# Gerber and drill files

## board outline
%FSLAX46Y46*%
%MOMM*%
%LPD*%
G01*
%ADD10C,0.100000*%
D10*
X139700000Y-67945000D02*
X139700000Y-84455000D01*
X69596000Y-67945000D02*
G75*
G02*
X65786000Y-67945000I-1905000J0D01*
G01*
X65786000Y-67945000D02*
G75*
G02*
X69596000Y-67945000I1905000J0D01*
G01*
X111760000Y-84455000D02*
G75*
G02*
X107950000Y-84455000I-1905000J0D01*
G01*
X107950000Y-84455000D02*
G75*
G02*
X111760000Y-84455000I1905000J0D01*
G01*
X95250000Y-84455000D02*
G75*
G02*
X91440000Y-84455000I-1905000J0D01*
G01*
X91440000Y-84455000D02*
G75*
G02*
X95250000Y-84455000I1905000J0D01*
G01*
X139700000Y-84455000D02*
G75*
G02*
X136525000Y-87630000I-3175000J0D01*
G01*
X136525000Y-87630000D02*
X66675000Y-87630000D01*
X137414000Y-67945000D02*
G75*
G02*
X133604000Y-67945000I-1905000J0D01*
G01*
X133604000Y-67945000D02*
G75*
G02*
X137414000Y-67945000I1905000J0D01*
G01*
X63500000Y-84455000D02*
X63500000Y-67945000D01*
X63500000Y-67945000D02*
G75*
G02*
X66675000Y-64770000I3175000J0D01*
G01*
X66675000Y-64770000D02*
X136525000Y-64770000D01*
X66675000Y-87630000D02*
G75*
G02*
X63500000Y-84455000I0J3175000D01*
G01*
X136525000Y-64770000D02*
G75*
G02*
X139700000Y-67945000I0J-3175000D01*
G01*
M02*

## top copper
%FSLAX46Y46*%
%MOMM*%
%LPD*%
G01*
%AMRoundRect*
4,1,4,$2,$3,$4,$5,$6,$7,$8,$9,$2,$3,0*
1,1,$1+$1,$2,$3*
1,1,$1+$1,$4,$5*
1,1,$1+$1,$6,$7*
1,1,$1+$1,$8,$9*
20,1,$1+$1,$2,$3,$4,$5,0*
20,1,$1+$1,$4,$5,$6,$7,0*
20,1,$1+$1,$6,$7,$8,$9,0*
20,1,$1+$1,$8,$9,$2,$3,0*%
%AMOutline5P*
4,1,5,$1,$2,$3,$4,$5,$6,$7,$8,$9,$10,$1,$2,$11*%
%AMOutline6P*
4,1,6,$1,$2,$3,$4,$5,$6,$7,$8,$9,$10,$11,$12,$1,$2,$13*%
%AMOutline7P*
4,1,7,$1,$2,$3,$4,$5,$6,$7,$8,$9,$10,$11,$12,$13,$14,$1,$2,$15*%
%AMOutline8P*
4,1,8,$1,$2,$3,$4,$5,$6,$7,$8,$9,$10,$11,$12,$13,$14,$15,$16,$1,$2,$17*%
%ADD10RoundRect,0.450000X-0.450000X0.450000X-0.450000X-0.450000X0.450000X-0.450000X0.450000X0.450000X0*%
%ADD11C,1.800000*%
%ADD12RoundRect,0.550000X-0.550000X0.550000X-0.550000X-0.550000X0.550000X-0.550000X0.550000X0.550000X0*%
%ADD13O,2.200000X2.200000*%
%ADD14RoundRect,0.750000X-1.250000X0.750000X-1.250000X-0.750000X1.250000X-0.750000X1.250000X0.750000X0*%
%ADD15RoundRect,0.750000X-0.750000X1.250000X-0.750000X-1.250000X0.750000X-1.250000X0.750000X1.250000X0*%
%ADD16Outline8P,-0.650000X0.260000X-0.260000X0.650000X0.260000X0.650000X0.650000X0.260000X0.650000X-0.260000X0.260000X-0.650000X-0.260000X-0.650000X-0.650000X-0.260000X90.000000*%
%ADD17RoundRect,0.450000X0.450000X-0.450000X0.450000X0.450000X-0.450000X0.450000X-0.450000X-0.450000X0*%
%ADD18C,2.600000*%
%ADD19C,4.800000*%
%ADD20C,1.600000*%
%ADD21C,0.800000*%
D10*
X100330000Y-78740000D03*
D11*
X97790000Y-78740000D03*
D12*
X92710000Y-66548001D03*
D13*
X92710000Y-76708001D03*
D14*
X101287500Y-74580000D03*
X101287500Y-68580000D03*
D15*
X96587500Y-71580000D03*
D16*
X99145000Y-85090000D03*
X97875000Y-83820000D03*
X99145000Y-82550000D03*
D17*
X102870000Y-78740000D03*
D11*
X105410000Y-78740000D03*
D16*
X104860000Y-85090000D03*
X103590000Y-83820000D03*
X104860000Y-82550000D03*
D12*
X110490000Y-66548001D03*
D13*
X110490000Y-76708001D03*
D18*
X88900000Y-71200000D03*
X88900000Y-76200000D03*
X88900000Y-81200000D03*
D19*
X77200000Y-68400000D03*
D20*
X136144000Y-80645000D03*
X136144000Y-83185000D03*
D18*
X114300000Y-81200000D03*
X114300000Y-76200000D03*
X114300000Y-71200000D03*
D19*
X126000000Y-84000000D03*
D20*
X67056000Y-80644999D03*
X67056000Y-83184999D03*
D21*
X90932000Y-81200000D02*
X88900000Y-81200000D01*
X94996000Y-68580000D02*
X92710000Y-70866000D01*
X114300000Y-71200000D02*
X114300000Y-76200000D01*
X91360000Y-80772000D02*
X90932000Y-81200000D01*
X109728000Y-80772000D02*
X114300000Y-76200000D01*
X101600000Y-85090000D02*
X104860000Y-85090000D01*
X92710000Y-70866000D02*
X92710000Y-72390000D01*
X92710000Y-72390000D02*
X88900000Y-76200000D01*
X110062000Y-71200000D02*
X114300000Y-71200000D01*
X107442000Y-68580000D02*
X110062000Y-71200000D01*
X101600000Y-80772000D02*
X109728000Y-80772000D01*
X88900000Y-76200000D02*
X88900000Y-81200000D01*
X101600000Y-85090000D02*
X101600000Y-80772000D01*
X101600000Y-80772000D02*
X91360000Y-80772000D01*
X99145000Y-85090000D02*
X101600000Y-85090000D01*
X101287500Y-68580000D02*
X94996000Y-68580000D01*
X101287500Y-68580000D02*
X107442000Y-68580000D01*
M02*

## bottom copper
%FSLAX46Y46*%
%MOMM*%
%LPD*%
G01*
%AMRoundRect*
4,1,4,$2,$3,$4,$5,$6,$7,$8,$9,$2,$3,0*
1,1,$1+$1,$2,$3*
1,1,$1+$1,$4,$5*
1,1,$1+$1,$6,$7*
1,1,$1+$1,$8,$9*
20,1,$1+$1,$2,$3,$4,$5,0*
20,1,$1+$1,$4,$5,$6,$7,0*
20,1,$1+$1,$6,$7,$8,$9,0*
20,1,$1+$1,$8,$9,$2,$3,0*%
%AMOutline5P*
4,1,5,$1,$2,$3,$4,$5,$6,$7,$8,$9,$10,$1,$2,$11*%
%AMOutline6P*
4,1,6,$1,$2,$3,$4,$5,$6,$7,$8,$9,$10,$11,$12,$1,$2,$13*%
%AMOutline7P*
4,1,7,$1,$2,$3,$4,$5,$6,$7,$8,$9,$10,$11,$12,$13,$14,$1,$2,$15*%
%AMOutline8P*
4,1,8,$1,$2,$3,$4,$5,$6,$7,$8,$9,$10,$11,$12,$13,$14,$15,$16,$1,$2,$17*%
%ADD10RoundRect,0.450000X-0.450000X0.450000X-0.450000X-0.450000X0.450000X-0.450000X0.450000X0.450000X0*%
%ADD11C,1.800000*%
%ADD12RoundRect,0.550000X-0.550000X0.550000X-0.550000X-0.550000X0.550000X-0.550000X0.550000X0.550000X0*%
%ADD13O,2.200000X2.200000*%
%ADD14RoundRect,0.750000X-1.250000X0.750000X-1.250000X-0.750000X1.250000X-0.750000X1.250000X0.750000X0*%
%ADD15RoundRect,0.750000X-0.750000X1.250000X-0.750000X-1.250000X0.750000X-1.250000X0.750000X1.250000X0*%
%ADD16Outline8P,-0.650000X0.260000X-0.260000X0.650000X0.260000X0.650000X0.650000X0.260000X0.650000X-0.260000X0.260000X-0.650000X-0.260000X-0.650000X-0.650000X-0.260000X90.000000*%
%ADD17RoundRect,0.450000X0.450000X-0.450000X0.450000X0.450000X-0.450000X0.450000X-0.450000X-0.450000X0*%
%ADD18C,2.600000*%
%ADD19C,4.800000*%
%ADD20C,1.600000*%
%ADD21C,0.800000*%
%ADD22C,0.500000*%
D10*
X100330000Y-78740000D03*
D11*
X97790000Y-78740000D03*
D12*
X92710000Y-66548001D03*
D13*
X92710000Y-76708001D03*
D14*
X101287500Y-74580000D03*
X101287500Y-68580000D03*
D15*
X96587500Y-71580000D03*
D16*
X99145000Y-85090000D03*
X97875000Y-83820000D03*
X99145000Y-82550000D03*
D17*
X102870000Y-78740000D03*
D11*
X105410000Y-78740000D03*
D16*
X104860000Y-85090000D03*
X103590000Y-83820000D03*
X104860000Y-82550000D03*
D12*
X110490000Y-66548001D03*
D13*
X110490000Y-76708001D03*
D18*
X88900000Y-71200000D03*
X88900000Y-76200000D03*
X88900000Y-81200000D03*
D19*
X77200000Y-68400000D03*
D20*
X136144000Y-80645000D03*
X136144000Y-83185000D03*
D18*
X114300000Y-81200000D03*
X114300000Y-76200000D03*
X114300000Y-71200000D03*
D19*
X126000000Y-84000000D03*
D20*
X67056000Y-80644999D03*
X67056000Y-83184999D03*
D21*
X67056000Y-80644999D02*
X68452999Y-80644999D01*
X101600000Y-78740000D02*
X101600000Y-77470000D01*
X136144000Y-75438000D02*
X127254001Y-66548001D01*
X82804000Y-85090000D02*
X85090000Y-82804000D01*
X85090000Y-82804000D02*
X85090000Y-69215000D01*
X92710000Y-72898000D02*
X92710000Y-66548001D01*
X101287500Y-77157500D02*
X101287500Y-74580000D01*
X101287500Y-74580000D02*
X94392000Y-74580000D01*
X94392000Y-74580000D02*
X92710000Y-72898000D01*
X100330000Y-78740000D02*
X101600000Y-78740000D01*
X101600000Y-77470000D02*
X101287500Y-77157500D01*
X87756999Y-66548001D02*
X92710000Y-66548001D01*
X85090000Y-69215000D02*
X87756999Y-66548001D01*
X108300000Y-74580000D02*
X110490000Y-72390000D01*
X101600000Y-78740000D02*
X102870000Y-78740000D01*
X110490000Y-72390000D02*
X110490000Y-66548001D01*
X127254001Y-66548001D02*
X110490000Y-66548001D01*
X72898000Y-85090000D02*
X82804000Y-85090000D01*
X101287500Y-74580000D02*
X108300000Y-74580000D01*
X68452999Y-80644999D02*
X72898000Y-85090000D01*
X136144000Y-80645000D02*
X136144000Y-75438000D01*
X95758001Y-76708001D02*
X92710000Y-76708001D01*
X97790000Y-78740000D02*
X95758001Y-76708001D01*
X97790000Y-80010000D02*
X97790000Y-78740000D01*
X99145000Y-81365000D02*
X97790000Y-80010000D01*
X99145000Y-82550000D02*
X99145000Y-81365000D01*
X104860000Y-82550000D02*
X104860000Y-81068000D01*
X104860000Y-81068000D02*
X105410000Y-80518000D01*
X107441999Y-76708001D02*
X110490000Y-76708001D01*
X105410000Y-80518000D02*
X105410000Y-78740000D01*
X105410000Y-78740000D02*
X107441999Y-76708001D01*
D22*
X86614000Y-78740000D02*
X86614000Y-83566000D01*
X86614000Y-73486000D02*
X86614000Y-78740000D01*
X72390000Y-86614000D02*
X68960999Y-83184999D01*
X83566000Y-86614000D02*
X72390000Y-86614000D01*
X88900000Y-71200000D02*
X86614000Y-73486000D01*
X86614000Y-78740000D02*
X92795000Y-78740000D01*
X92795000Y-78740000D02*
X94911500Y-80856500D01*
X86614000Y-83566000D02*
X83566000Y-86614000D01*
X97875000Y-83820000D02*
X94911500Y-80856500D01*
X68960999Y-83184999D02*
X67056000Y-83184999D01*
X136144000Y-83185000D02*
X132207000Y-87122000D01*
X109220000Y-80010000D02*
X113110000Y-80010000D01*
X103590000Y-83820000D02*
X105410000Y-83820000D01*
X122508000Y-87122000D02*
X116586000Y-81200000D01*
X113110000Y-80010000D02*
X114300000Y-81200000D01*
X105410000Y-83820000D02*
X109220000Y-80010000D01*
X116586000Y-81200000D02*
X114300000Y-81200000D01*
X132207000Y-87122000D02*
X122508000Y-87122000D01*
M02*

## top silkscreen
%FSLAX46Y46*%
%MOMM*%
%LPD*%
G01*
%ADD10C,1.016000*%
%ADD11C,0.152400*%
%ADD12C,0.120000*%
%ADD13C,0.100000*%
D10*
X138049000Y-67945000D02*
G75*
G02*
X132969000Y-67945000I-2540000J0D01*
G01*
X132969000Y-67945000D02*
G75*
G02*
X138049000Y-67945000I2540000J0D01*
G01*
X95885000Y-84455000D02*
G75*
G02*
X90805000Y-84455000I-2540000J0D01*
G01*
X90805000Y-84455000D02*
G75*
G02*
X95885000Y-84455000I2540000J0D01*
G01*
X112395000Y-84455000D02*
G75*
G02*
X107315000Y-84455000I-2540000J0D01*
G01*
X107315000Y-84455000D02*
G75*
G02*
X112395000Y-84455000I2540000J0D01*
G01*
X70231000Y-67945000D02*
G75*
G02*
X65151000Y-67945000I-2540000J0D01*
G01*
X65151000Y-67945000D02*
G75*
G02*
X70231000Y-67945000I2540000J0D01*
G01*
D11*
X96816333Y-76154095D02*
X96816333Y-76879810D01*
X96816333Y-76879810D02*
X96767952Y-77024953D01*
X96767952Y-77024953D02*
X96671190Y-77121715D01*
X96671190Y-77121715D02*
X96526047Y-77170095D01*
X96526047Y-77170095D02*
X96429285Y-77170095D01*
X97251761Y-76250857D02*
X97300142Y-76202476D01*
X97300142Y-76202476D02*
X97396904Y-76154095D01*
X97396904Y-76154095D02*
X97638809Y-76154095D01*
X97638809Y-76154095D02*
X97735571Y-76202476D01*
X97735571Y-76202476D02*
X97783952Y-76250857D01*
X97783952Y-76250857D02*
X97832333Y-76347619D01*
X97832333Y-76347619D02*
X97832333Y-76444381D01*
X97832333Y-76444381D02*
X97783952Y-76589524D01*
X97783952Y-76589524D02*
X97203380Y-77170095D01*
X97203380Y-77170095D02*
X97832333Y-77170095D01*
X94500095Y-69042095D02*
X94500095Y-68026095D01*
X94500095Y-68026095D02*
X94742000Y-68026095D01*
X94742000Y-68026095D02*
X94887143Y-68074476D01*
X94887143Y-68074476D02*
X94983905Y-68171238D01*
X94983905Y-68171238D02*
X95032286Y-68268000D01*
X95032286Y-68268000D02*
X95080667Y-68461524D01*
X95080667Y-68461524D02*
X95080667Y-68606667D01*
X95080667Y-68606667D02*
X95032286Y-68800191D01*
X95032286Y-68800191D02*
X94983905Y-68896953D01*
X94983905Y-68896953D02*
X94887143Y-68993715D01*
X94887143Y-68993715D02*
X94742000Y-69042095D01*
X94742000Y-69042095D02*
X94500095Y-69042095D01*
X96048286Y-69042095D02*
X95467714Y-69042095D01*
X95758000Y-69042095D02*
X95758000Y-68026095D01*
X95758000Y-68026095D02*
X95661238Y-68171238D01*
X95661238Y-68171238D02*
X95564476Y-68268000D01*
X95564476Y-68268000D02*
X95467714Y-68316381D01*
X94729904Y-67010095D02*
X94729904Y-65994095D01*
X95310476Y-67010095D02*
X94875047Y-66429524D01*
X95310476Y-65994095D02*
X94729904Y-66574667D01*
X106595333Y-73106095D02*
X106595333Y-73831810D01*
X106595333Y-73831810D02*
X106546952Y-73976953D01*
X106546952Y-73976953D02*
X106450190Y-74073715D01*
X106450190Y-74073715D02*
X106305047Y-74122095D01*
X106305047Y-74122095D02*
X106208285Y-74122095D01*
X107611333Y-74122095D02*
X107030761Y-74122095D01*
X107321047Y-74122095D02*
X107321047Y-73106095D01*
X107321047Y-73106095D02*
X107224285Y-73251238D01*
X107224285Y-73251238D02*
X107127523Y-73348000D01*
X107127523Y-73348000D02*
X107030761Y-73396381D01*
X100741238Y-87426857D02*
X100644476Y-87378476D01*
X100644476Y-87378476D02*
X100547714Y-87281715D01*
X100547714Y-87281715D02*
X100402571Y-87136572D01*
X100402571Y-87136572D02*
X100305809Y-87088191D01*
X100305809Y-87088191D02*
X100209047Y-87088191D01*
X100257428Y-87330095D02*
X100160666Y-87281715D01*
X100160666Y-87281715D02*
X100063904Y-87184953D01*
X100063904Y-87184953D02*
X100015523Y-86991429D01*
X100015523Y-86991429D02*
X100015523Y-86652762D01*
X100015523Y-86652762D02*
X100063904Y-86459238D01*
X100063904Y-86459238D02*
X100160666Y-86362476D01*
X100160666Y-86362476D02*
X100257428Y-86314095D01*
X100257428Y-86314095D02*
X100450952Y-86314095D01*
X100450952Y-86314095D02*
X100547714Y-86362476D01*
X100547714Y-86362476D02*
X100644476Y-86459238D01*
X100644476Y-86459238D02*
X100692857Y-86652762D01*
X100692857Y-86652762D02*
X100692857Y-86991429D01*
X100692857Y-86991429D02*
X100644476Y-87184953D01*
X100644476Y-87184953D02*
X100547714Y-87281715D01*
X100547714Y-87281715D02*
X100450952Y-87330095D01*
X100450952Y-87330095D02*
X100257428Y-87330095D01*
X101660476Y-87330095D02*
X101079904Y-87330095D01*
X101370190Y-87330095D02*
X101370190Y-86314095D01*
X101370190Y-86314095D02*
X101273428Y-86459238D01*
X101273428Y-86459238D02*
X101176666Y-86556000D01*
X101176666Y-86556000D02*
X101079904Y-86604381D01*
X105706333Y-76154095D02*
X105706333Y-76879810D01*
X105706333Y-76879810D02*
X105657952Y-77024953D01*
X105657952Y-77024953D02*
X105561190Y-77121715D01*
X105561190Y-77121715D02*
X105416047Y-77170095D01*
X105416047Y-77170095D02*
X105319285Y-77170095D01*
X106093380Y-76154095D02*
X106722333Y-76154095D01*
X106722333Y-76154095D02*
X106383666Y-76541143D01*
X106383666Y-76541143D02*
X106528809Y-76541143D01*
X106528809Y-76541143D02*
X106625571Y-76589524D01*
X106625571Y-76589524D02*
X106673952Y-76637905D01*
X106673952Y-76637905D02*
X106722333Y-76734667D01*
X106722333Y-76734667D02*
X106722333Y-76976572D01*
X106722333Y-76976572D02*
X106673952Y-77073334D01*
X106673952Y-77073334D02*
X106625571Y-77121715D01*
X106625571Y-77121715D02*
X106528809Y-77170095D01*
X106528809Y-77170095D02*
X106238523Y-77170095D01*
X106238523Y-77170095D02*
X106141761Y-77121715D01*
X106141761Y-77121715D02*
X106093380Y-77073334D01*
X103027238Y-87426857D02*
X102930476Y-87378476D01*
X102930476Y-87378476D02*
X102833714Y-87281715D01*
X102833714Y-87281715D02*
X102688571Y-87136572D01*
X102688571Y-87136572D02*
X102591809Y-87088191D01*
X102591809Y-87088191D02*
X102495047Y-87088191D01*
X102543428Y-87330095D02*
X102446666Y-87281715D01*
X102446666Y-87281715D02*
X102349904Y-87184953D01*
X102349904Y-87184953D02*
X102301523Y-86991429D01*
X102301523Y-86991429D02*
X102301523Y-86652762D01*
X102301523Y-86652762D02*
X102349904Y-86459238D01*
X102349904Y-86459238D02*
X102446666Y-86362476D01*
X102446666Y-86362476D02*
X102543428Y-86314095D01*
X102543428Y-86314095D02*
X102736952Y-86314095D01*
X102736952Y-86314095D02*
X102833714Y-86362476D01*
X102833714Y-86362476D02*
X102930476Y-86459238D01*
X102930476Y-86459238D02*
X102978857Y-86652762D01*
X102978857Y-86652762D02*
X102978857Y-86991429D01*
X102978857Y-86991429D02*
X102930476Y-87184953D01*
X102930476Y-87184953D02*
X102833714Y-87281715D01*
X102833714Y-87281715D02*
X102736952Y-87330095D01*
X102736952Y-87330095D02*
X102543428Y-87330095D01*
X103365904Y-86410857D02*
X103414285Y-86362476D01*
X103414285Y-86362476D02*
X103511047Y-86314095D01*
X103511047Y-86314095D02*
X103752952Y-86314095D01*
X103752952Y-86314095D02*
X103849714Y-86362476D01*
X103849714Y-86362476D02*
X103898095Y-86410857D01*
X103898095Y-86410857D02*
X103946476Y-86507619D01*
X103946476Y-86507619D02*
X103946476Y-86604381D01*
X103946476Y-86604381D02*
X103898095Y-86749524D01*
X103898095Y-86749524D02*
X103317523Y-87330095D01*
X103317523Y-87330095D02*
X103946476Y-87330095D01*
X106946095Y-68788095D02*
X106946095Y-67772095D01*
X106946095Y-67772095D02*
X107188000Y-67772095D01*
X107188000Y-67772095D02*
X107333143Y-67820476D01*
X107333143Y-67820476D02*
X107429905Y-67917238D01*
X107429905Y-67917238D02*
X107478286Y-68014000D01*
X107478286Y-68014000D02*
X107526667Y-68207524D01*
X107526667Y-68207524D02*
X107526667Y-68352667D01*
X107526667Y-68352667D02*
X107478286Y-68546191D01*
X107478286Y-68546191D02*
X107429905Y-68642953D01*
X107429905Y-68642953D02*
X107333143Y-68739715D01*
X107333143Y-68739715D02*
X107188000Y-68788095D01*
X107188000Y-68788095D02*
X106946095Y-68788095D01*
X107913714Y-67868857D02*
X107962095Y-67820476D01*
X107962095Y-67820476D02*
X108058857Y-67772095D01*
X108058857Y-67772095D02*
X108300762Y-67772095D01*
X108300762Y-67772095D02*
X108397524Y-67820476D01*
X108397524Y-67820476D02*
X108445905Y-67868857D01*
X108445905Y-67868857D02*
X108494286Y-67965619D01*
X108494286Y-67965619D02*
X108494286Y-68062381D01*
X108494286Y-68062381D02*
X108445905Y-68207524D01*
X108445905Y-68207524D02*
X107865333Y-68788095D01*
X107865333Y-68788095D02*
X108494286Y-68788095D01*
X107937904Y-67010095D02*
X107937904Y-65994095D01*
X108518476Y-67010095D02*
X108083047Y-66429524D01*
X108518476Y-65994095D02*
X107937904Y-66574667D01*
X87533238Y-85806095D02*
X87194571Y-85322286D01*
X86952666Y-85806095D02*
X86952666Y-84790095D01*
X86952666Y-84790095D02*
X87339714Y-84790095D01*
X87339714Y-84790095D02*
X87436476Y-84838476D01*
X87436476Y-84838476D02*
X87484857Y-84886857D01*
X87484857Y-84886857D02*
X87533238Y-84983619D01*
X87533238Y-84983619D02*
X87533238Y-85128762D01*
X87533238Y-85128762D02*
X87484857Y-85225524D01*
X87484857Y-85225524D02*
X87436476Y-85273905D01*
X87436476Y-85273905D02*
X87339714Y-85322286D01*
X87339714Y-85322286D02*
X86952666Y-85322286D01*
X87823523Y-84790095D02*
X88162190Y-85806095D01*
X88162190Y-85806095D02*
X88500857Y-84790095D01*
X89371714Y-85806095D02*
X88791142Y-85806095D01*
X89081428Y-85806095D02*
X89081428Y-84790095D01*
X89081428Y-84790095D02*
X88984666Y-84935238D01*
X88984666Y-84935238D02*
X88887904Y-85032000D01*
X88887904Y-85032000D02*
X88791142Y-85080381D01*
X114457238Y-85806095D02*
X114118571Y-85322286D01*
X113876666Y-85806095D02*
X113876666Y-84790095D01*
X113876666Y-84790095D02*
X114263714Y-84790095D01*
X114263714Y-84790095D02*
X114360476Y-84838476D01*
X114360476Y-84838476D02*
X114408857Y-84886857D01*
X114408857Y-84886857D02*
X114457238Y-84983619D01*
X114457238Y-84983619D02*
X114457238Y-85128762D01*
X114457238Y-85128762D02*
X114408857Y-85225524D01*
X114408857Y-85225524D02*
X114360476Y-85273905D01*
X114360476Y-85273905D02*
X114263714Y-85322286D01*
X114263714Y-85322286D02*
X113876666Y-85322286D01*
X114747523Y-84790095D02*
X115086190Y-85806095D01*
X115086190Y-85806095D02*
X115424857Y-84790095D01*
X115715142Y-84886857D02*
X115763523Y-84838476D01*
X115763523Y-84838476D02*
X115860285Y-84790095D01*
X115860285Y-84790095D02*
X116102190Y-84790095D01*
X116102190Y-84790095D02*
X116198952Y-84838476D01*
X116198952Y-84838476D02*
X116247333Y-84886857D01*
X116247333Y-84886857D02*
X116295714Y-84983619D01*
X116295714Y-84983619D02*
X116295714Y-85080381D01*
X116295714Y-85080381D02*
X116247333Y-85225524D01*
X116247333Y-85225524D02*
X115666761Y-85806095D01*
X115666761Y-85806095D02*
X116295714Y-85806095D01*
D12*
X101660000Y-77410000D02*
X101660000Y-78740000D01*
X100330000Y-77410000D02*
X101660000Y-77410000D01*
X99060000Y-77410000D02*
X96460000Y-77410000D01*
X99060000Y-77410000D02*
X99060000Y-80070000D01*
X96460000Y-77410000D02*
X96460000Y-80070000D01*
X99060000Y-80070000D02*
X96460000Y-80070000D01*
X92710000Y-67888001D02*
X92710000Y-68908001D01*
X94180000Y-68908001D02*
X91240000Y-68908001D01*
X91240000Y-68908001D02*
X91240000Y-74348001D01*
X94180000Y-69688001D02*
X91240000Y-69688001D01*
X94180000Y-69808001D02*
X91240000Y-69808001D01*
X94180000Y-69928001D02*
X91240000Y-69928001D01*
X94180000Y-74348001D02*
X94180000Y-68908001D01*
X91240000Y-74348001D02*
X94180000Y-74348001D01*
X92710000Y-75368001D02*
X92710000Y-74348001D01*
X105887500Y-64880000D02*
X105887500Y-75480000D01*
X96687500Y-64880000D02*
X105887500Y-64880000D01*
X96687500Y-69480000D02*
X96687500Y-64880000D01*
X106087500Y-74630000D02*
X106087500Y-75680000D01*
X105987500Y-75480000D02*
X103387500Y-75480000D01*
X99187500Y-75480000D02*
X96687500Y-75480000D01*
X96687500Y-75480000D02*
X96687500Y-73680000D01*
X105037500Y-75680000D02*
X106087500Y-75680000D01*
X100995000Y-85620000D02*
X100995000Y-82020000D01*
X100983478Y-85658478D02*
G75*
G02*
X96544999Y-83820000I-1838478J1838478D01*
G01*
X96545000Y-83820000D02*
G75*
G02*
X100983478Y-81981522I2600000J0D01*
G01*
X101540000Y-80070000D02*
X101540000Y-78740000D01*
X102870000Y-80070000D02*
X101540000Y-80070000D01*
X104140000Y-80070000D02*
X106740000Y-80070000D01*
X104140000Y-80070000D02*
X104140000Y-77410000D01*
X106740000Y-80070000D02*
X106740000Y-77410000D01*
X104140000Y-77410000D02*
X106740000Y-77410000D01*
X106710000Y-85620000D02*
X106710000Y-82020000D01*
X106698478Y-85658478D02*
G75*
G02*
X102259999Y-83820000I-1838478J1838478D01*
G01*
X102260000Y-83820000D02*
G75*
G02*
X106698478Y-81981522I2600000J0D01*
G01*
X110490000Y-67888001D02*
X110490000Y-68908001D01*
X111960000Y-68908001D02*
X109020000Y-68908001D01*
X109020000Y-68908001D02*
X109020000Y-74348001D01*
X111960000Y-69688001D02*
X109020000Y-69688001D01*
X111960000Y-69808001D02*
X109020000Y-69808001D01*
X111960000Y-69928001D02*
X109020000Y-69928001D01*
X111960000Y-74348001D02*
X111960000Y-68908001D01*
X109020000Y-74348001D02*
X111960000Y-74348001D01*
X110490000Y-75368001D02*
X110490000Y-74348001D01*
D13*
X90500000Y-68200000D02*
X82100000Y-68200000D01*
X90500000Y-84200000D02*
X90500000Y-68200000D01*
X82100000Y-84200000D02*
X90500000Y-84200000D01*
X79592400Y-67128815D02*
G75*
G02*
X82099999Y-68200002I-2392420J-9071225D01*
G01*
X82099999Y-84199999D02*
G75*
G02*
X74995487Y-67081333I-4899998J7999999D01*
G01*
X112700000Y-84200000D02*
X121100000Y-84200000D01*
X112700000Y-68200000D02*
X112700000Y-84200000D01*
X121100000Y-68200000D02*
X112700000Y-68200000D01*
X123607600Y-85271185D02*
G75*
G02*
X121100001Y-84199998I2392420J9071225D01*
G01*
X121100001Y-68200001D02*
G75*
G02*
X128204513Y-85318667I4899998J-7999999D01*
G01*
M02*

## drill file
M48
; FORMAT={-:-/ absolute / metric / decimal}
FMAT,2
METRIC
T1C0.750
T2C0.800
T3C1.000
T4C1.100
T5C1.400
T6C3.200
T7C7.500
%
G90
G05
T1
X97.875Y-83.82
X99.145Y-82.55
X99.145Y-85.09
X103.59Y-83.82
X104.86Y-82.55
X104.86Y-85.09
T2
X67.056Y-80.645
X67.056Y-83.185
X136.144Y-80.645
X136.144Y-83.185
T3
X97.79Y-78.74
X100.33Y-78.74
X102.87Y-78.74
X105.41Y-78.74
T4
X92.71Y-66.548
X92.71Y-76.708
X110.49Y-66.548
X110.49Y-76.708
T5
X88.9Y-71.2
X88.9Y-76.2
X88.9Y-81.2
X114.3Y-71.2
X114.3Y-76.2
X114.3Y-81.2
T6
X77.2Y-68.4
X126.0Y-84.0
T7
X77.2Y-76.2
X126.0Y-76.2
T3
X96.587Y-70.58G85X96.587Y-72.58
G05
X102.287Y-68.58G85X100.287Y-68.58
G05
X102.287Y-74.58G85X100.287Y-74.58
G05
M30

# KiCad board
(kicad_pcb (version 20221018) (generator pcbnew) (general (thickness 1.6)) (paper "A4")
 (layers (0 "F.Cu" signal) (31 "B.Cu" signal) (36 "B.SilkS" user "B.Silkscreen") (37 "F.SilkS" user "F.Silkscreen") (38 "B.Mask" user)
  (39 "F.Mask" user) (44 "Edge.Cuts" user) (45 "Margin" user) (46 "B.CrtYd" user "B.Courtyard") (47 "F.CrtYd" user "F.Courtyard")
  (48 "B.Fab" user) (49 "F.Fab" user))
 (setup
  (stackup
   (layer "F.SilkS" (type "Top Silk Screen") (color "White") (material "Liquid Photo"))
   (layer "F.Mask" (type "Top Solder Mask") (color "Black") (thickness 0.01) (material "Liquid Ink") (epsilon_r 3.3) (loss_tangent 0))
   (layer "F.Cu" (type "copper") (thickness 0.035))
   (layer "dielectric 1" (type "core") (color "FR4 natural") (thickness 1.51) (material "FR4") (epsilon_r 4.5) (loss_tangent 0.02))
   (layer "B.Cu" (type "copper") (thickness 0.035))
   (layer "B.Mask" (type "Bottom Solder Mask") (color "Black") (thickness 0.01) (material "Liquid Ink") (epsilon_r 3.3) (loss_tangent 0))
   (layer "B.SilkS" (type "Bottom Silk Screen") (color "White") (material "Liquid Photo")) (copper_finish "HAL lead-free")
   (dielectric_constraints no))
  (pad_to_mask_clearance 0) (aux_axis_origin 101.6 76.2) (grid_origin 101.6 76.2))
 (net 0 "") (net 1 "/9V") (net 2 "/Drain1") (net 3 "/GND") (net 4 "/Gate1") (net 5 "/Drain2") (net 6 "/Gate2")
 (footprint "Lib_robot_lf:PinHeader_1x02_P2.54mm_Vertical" (layer "F.Cu") (at 100.33 78.74 -90)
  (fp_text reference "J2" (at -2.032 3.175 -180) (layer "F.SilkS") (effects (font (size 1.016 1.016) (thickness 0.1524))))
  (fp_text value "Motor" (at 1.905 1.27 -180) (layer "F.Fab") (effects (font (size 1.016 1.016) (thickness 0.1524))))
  (fp_line (start -1.33 -1.33) (end 0 -1.33) (stroke (width 0.12) (type solid)) (layer "F.SilkS"))
  (fp_line (start -1.33 0) (end -1.33 -1.33) (stroke (width 0.12) (type solid)) (layer "F.SilkS"))
  (fp_line (start -1.33 1.27) (end -1.33 3.87) (stroke (width 0.12) (type solid)) (layer "F.SilkS"))
  (fp_line (start -1.33 1.27) (end 1.33 1.27) (stroke (width 0.12) (type solid)) (layer "F.SilkS"))
  (fp_line (start -1.33 3.87) (end 1.33 3.87) (stroke (width 0.12) (type solid)) (layer "F.SilkS"))
  (fp_line (start 1.33 1.27) (end 1.33 3.87) (stroke (width 0.12) (type solid)) (layer "F.SilkS"))
  (pad "1" thru_hole roundrect (at 0 0 270) (size 1.8 1.8) (drill 1) (layers "*.Cu" "*.Mask") (roundrect_rratio 0.25) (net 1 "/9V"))
  (pad "2" thru_hole circle (at 0 2.54 270) (size 1.8 1.8) (drill 1) (layers "*.Cu" "*.Mask") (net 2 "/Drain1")))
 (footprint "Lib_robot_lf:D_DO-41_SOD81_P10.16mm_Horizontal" (layer "F.Cu") (at 92.71 66.548001 -90)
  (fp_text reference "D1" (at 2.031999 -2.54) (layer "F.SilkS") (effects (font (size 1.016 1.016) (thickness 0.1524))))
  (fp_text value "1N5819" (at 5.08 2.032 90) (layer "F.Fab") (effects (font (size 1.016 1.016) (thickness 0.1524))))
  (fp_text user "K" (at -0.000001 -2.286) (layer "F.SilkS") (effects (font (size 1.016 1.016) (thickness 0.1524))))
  (fp_line (start 1.34 0) (end 2.36 0) (stroke (width 0.12) (type solid)) (layer "F.SilkS"))
  (fp_line (start 2.36 -1.47) (end 2.36 1.47) (stroke (width 0.12) (type solid)) (layer "F.SilkS"))
  (fp_line (start 2.36 1.47) (end 7.8 1.47) (stroke (width 0.12) (type solid)) (layer "F.SilkS"))
  (fp_line (start 3.14 -1.47) (end 3.14 1.47) (stroke (width 0.12) (type solid)) (layer "F.SilkS"))
  (fp_line (start 3.26 -1.47) (end 3.26 1.47) (stroke (width 0.12) (type solid)) (layer "F.SilkS"))
  (fp_line (start 3.38 -1.47) (end 3.38 1.47) (stroke (width 0.12) (type solid)) (layer "F.SilkS"))
  (fp_line (start 7.8 -1.47) (end 2.36 -1.47) (stroke (width 0.12) (type solid)) (layer "F.SilkS"))
  (fp_line (start 7.8 1.47) (end 7.8 -1.47) (stroke (width 0.12) (type solid)) (layer "F.SilkS"))
  (fp_line (start 8.82 0) (end 7.8 0) (stroke (width 0.12) (type solid)) (layer "F.SilkS"))
  (pad "1" thru_hole roundrect (at 0 0 270) (size 2.2 2.2) (drill 1.1) (layers "*.Cu" "*.Mask") (roundrect_rratio 0.25) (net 1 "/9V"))
  (pad "2" thru_hole oval (at 10.16 0 270) (size 2.2 2.2) (drill 1.1) (layers "*.Cu" "*.Mask") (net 2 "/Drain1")))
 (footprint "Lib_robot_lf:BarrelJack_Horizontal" (layer "F.Cu") (at 101.2875 74.58 -90)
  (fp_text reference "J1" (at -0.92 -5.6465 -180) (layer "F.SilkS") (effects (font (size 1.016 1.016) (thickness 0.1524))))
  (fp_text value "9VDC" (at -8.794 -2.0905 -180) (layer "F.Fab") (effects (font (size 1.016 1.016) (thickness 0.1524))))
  (fp_line (start -9.7 -4.6) (end 0.9 -4.6) (stroke (width 0.12) (type solid)) (layer "F.SilkS"))
  (fp_line (start -9.7 4.6) (end -9.7 -4.6) (stroke (width 0.12) (type solid)) (layer "F.SilkS"))
  (fp_line (start -5.1 4.6) (end -9.7 4.6) (stroke (width 0.12) (type solid)) (layer "F.SilkS"))
  (fp_line (start 0.05 -4.8) (end 1.1 -4.8) (stroke (width 0.12) (type solid)) (layer "F.SilkS"))
  (fp_line (start 0.9 -4.7) (end 0.9 -2.1) (stroke (width 0.12) (type solid)) (layer "F.SilkS"))
  (fp_line (start 0.9 2.1) (end 0.9 4.6) (stroke (width 0.12) (type solid)) (layer "F.SilkS"))
  (fp_line (start 0.9 4.6) (end -0.9 4.6) (stroke (width 0.12) (type solid)) (layer "F.SilkS"))
  (fp_line (start 1.1 -3.75) (end 1.1 -4.8) (stroke (width 0.12) (type solid)) (layer "F.SilkS"))
  (pad "1" thru_hole roundrect (at 0 0 270) (size 3 4) (drill oval 1 3) (layers "*.Cu" "*.Mask") (roundrect_rratio 0.25) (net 1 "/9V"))
  (pad "2" thru_hole roundrect (at -6 0 270) (size 3 4) (drill oval 1 3) (layers "*.Cu" "*.Mask") (roundrect_rratio 0.25) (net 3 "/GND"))
  (pad "3" thru_hole roundrect (at -3 4.7 270) (size 4 3) (drill oval 3 1) (layers "*.Cu" "*.Mask") (roundrect_rratio 0.25)))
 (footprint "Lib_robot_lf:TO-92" (layer "F.Cu") (at 99.145 85.09 90)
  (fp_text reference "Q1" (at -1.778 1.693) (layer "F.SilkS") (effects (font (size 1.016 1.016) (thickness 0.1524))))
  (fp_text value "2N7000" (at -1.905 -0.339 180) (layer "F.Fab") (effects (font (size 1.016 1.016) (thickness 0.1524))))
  (fp_line (start -0.53 1.85) (end 3.07 1.85) (stroke (width 0.12) (type solid)) (layer "F.SilkS"))
  (fp_arc (start -0.568478 1.838478) (mid -1.132087 -0.994977) (end 1.27 -2.6) (stroke (width 0.12) (type solid)) (layer "F.SilkS"))
  (fp_arc (start 1.27 -2.6) (mid 3.672087 -0.994977) (end 3.108478 1.838478) (stroke (width 0.12) (type solid)) (layer "F.SilkS"))
  (pad "1" thru_hole roundrect (at 0 0 90) (size 1.3 1.3) (drill 0.75) (layers "*.Cu" "*.Mask") (roundrect_rratio 0) (chamfer_ratio 0.3)
   (chamfer top_left top_right bottom_left bottom_right) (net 3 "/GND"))
  (pad "2" thru_hole roundrect (at 1.27 -1.27 90) (size 1.3 1.3) (drill 0.75) (layers "*.Cu" "*.Mask") (roundrect_rratio 0)
   (chamfer_ratio 0.3) (chamfer top_left top_right bottom_left bottom_right) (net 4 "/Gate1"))
  (pad "3" thru_hole roundrect (at 2.54 0 90) (size 1.3 1.3) (drill 0.75) (layers "*.Cu" "*.Mask") (roundrect_rratio 0) (chamfer_ratio 0.3)
   (chamfer top_left top_right bottom_left bottom_right) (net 2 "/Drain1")))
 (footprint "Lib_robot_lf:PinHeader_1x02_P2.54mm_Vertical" (layer "F.Cu") (at 102.87 78.74 90)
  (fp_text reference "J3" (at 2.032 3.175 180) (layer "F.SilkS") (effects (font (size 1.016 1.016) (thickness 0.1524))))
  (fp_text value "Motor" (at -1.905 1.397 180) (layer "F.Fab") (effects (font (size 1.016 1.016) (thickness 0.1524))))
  (fp_line (start -1.33 -1.33) (end 0 -1.33) (stroke (width 0.12) (type solid)) (layer "F.SilkS"))
  (fp_line (start -1.33 0) (end -1.33 -1.33) (stroke (width 0.12) (type solid)) (layer "F.SilkS"))
  (fp_line (start -1.33 1.27) (end -1.33 3.87) (stroke (width 0.12) (type solid)) (layer "F.SilkS"))
  (fp_line (start -1.33 1.27) (end 1.33 1.27) (stroke (width 0.12) (type solid)) (layer "F.SilkS"))
  (fp_line (start -1.33 3.87) (end 1.33 3.87) (stroke (width 0.12) (type solid)) (layer "F.SilkS"))
  (fp_line (start 1.33 1.27) (end 1.33 3.87) (stroke (width 0.12) (type solid)) (layer "F.SilkS"))
  (pad "1" thru_hole roundrect (at 0 0 90) (size 1.8 1.8) (drill 1) (layers "*.Cu" "*.Mask") (roundrect_rratio 0.25) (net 1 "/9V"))
  (pad "2" thru_hole circle (at 0 2.54 90) (size 1.8 1.8) (drill 1) (layers "*.Cu" "*.Mask") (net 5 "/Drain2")))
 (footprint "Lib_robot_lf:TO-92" (layer "F.Cu") (at 104.86 85.09 90)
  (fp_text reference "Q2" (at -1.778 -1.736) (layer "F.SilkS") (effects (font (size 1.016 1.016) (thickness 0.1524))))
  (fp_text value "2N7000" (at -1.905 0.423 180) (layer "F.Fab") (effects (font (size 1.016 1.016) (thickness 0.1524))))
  (fp_line (start -0.53 1.85) (end 3.07 1.85) (stroke (width 0.12) (type solid)) (layer "F.SilkS"))
  (fp_arc (start -0.568478 1.838478) (mid -1.132087 -0.994977) (end 1.27 -2.6) (stroke (width 0.12) (type solid)) (layer "F.SilkS"))
  (fp_arc (start 1.27 -2.6) (mid 3.672087 -0.994977) (end 3.108478 1.838478) (stroke (width 0.12) (type solid)) (layer "F.SilkS"))
  (pad "1" thru_hole roundrect (at 0 0 90) (size 1.3 1.3) (drill 0.75) (layers "*.Cu" "*.Mask") (roundrect_rratio 0) (chamfer_ratio 0.3)
   (chamfer top_left top_right bottom_left bottom_right) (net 3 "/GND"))
  (pad "2" thru_hole roundrect (at 1.27 -1.27 90) (size 1.3 1.3) (drill 0.75) (layers "*.Cu" "*.Mask") (roundrect_rratio 0)
   (chamfer_ratio 0.3) (chamfer top_left top_right bottom_left bottom_right) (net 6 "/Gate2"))
  (pad "3" thru_hole roundrect (at 2.54 0 90) (size 1.3 1.3) (drill 0.75) (layers "*.Cu" "*.Mask") (roundrect_rratio 0) (chamfer_ratio 0.3)
   (chamfer top_left top_right bottom_left bottom_right) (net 5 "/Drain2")))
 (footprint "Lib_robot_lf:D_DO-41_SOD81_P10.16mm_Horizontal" (layer "F.Cu") (at 110.49 66.548001 -90)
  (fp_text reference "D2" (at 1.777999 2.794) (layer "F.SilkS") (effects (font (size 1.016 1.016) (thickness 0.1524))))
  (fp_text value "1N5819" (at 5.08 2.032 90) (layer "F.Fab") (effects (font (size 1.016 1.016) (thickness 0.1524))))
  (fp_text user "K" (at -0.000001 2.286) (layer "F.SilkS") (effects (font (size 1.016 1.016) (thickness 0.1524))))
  (fp_line (start 1.34 0) (end 2.36 0) (stroke (width 0.12) (type solid)) (layer "F.SilkS"))
  (fp_line (start 2.36 -1.47) (end 2.36 1.47) (stroke (width 0.12) (type solid)) (layer "F.SilkS"))
  (fp_line (start 2.36 1.47) (end 7.8 1.47) (stroke (width 0.12) (type solid)) (layer "F.SilkS"))
  (fp_line (start 3.14 -1.47) (end 3.14 1.47) (stroke (width 0.12) (type solid)) (layer "F.SilkS"))
  (fp_line (start 3.26 -1.47) (end 3.26 1.47) (stroke (width 0.12) (type solid)) (layer "F.SilkS"))
  (fp_line (start 3.38 -1.47) (end 3.38 1.47) (stroke (width 0.12) (type solid)) (layer "F.SilkS"))
  (fp_line (start 7.8 -1.47) (end 2.36 -1.47) (stroke (width 0.12) (type solid)) (layer "F.SilkS"))
  (fp_line (start 7.8 1.47) (end 7.8 -1.47) (stroke (width 0.12) (type solid)) (layer "F.SilkS"))
  (fp_line (start 8.82 0) (end 7.8 0) (stroke (width 0.12) (type solid)) (layer "F.SilkS"))
  (pad "1" thru_hole roundrect (at 0 0 270) (size 2.2 2.2) (drill 1.1) (layers "*.Cu" "*.Mask") (roundrect_rratio 0.25) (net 1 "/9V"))
  (pad "2" thru_hole oval (at 10.16 0 270) (size 2.2 2.2) (drill 1.1) (layers "*.Cu" "*.Mask") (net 5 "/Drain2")))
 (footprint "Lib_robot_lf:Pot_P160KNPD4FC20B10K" (layer "B.Cu") (at 88.9 76.2 -90)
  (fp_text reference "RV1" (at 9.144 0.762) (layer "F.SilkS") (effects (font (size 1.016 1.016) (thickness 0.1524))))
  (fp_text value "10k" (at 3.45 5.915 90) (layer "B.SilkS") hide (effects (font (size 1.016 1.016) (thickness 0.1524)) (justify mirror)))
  (fp_line (start -8 -1.6) (end -8 6.8) (stroke (width 0.1) (type default)) (layer "F.SilkS"))
  (fp_line (start 8 -1.6) (end -8 -1.6) (stroke (width 0.1) (type default)) (layer "F.SilkS"))
  (fp_line (start 8 6.8) (end 8 -1.6) (stroke (width 0.1) (type default)) (layer "F.SilkS"))
  (fp_arc (start -9.071185 9.3076) (mid -8.627186 8.014674) (end -7.999999 6.800001) (stroke (width 0.1) (type default)) (layer "F.SilkS"))
  (fp_arc (start 7.999999 6.800001) (mid 3.596022 20.364789) (end -9.118667 13.904513) (stroke (width 0.1) (type default)) (layer "F.SilkS"))
  (pad "" np_thru_hole circle (at 0 11.7 270) (size 7.5 7.5) (drill 7.5) (layers "*.Cu" "*.Mask"))
  (pad "1" thru_hole circle (at -5 0 270) (size 2.6 2.6) (drill 1.4) (layers "*.Cu" "*.Mask") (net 4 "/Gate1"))
  (pad "2" thru_hole circle (at 0 0 270) (size 2.6 2.6) (drill 1.4) (layers "*.Cu" "*.Mask") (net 3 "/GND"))
  (pad "3" thru_hole circle (at 5 0 270) (size 2.6 2.6) (drill 1.4) (layers "*.Cu" "*.Mask") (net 3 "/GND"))
  (pad "MH1" thru_hole circle (at -7.8 11.7 270) (size 4.8 4.8) (drill 3.2) (layers "*.Cu" "*.Mask")))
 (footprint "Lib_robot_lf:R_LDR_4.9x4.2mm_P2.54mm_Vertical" (layer "B.Cu") (at 136.144 80.645 -90)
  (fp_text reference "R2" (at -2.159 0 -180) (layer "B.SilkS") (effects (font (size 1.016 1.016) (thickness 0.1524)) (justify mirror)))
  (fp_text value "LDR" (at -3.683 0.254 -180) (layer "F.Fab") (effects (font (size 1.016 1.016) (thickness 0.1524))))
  (pad "1" thru_hole circle (at 0 0 270) (size 1.6 1.6) (drill 0.8) (layers "*.Cu" "*.Mask") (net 1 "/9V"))
  (pad "2" thru_hole circle (at 2.54 0 270) (size 1.6 1.6) (drill 0.8) (layers "*.Cu" "*.Mask") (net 6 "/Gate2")))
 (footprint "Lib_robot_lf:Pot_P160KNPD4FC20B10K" (layer "B.Cu") (at 114.3 76.2 90)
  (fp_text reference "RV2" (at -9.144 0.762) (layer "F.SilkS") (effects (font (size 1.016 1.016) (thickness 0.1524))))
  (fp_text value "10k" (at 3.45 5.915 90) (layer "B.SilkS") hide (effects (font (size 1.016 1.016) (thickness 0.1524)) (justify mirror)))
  (fp_line (start -8 -1.6) (end -8 6.8) (stroke (width 0.1) (type default)) (layer "F.SilkS"))
  (fp_line (start 8 -1.6) (end -8 -1.6) (stroke (width 0.1) (type default)) (layer "F.SilkS"))
  (fp_line (start 8 6.8) (end 8 -1.6) (stroke (width 0.1) (type default)) (layer "F.SilkS"))
  (fp_arc (start -9.071185 9.3076) (mid -8.627186 8.014674) (end -7.999999 6.800001) (stroke (width 0.1) (type default)) (layer "F.SilkS"))
  (fp_arc (start 7.999999 6.800001) (mid 3.596022 20.364789) (end -9.118667 13.904513) (stroke (width 0.1) (type default)) (layer "F.SilkS"))
  (pad "" np_thru_hole circle (at 0 11.7 90) (size 7.5 7.5) (drill 7.5) (layers "*.Cu" "*.Mask"))
  (pad "1" thru_hole circle (at -5 0 90) (size 2.6 2.6) (drill 1.4) (layers "*.Cu" "*.Mask") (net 6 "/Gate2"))
  (pad "2" thru_hole circle (at 0 0 90) (size 2.6 2.6) (drill 1.4) (layers "*.Cu" "*.Mask") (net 3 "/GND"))
  (pad "3" thru_hole circle (at 5 0 90) (size 2.6 2.6) (drill 1.4) (layers "*.Cu" "*.Mask") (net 3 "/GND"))
  (pad "MH1" thru_hole circle (at -7.8 11.7 90) (size 4.8 4.8) (drill 3.2) (layers "*.Cu" "*.Mask")))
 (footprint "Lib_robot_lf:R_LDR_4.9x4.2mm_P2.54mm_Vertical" (layer "B.Cu") (at 67.056 80.644999 -90)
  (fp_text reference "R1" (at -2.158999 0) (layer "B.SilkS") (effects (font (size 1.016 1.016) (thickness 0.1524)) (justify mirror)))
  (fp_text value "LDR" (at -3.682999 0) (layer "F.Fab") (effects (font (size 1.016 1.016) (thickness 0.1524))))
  (pad "1" thru_hole circle (at 0 0 270) (size 1.6 1.6) (drill 0.8) (layers "*.Cu" "*.Mask") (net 1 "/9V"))
  (pad "2" thru_hole circle (at 2.54 0 270) (size 1.6 1.6) (drill 0.8) (layers "*.Cu" "*.Mask") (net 4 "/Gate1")))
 (gr_circle (center 135.509 67.945) (end 138.049 67.945) (stroke (width 1.016) (type default)) (fill none) (layer "F.SilkS"))
 (gr_circle (center 93.345 84.455) (end 95.885 84.455) (stroke (width 1.016) (type default)) (fill none) (layer "F.SilkS"))
 (gr_circle (center 109.855 84.455) (end 112.395 84.455) (stroke (width 1.016) (type default)) (fill none) (layer "F.SilkS"))
 (gr_circle (center 67.691 67.945) (end 70.231 67.945) (stroke (width 1.016) (type default)) (fill none) (layer "F.SilkS"))
 (gr_line (start 139.7 67.945) (end 139.7 84.455) (stroke (width 0.1) (type default)) (layer "Edge.Cuts"))
 (gr_circle (center 67.691 67.945) (end 65.786 67.945) (stroke (width 0.1) (type default)) (fill none) (layer "Edge.Cuts"))
 (gr_circle (center 109.855 84.455) (end 109.855 86.36) (stroke (width 0.1) (type default)) (fill none) (layer "Edge.Cuts"))
 (gr_circle (center 93.345 84.455) (end 93.345 86.36) (stroke (width 0.1) (type default)) (fill none) (layer "Edge.Cuts"))
 (gr_arc (start 139.7 84.455) (mid 138.770064 86.700064) (end 136.525 87.63) (stroke (width 0.1) (type default)) (layer "Edge.Cuts"))
 (gr_line (start 136.525 87.63) (end 66.675 87.63) (stroke (width 0.1) (type default)) (layer "Edge.Cuts"))
 (gr_circle (center 135.509 67.945) (end 137.414 67.945) (stroke (width 0.1) (type default)) (fill none) (layer "Edge.Cuts"))
 (gr_line (start 63.5 84.455) (end 63.5 67.945) (stroke (width 0.1) (type default)) (layer "Edge.Cuts"))
 (gr_arc (start 63.5 67.945) (mid 64.429936 65.699936) (end 66.675 64.77) (stroke (width 0.1) (type default)) (layer "Edge.Cuts"))
 (gr_line (start 66.675 64.77) (end 136.525 64.77) (stroke (width 0.1) (type default)) (layer "Edge.Cuts"))
 (gr_arc (start 66.675 87.63) (mid 64.429936 86.700064) (end 63.5 84.455) (stroke (width 0.1) (type default)) (layer "Edge.Cuts"))
 (gr_arc (start 136.525 64.77) (mid 138.770064 65.699936) (end 139.7 67.945) (stroke (width 0.1) (type default)) (layer "Edge.Cuts"))
 (segment (start 67.056 80.644999) (end 68.452999 80.644999) (width 0.8) (layer "B.Cu") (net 1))
 (segment (start 101.6 78.74) (end 101.6 77.47) (width 0.8) (layer "B.Cu") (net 1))
 (segment (start 136.144 75.438) (end 127.254001 66.548001) (width 0.8) (layer "B.Cu") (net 1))
 (segment (start 82.804 85.09) (end 85.09 82.804) (width 0.8) (layer "B.Cu") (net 1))
 (segment (start 85.09 82.804) (end 85.09 69.215) (width 0.8) (layer "B.Cu") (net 1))
 (segment (start 92.71 72.898) (end 92.71 66.548001) (width 0.8) (layer "B.Cu") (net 1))
 (segment (start 101.2875 77.1575) (end 101.2875 74.58) (width 0.8) (layer "B.Cu") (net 1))
 (segment (start 101.2875 74.58) (end 94.392 74.58) (width 0.8) (layer "B.Cu") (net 1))
 (segment (start 94.392 74.58) (end 92.71 72.898) (width 0.8) (layer "B.Cu") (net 1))
 (segment (start 100.33 78.74) (end 101.6 78.74) (width 0.8) (layer "B.Cu") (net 1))
 (segment (start 101.6 77.47) (end 101.2875 77.1575) (width 0.8) (layer "B.Cu") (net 1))
 (segment (start 87.756999 66.548001) (end 92.71 66.548001) (width 0.8) (layer "B.Cu") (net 1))
 (segment (start 85.09 69.215) (end 87.756999 66.548001) (width 0.8) (layer "B.Cu") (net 1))
 (segment (start 108.3 74.58) (end 110.49 72.39) (width 0.8) (layer "B.Cu") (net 1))
 (segment (start 101.6 78.74) (end 102.87 78.74) (width 0.8) (layer "B.Cu") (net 1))
 (segment (start 110.49 72.39) (end 110.49 66.548001) (width 0.8) (layer "B.Cu") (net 1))
 (segment (start 127.254001 66.548001) (end 110.49 66.548001) (width 0.8) (layer "B.Cu") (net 1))
 (segment (start 72.898 85.09) (end 82.804 85.09) (width 0.8) (layer "B.Cu") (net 1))
 (segment (start 101.2875 74.58) (end 108.3 74.58) (width 0.8) (layer "B.Cu") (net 1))
 (segment (start 68.452999 80.644999) (end 72.898 85.09) (width 0.8) (layer "B.Cu") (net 1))
 (segment (start 136.144 80.645) (end 136.144 75.438) (width 0.8) (layer "B.Cu") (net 1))
 (segment (start 95.758001 76.708001) (end 92.71 76.708001) (width 0.8) (layer "B.Cu") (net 2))
 (segment (start 97.79 78.74) (end 95.758001 76.708001) (width 0.8) (layer "B.Cu") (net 2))
 (segment (start 97.79 80.01) (end 97.79 78.74) (width 0.8) (layer "B.Cu") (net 2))
 (segment (start 99.145 81.365) (end 97.79 80.01) (width 0.8) (layer "B.Cu") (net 2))
 (segment (start 99.145 82.55) (end 99.145 81.365) (width 0.8) (layer "B.Cu") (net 2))
 (segment (start 104.86 82.55) (end 104.86 81.068) (width 0.8) (layer "B.Cu") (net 5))
 (segment (start 104.86 81.068) (end 105.41 80.518) (width 0.8) (layer "B.Cu") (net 5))
 (segment (start 107.441999 76.708001) (end 110.49 76.708001) (width 0.8) (layer "B.Cu") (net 5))
 (segment (start 105.41 80.518) (end 105.41 78.74) (width 0.8) (layer "B.Cu") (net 5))
 (segment (start 105.41 78.74) (end 107.441999 76.708001) (width 0.8) (layer "B.Cu") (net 5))
 (segment (start 90.932 81.2) (end 88.9 81.2) (width 0.8) (layer "F.Cu") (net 3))
 (segment (start 94.996 68.58) (end 92.71 70.866) (width 0.8) (layer "F.Cu") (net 3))
 (segment (start 114.3 71.2) (end 114.3 76.2) (width 0.8) (layer "F.Cu") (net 3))
 (segment (start 91.36 80.772) (end 90.932 81.2) (width 0.8) (layer "F.Cu") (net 3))
 (segment (start 109.728 80.772) (end 114.3 76.2) (width 0.8) (layer "F.Cu") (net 3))
 (segment (start 101.6 85.09) (end 104.86 85.09) (width 0.8) (layer "F.Cu") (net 3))
 (segment (start 92.71 70.866) (end 92.71 72.39) (width 0.8) (layer "F.Cu") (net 3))
 (segment (start 92.71 72.39) (end 88.9 76.2) (width 0.8) (layer "F.Cu") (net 3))
 (segment (start 110.062 71.2) (end 114.3 71.2) (width 0.8) (layer "F.Cu") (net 3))
 (segment (start 107.442 68.58) (end 110.062 71.2) (width 0.8) (layer "F.Cu") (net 3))
 (segment (start 101.6 80.772) (end 109.728 80.772) (width 0.8) (layer "F.Cu") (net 3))
 (segment (start 88.9 76.2) (end 88.9 81.2) (width 0.8) (layer "F.Cu") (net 3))
 (segment (start 101.6 85.09) (end 101.6 80.772) (width 0.8) (layer "F.Cu") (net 3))
 (segment (start 101.6 80.772) (end 91.36 80.772) (width 0.8) (layer "F.Cu") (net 3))
 (segment (start 99.145 85.09) (end 101.6 85.09) (width 0.8) (layer "F.Cu") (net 3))
 (segment (start 101.2875 68.58) (end 94.996 68.58) (width 0.8) (layer "F.Cu") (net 3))
 (segment (start 101.2875 68.58) (end 107.442 68.58) (width 0.8) (layer "F.Cu") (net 3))
 (segment (start 86.614 78.74) (end 86.614 83.566) (width 0.5) (layer "B.Cu") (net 4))
 (segment (start 86.614 73.486) (end 86.614 78.74) (width 0.5) (layer "B.Cu") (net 4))
 (segment (start 72.39 86.614) (end 68.960999 83.184999) (width 0.5) (layer "B.Cu") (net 4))
 (segment (start 83.566 86.614) (end 72.39 86.614) (width 0.5) (layer "B.Cu") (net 4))
 (segment (start 88.9 71.2) (end 86.614 73.486) (width 0.5) (layer "B.Cu") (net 4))
 (segment (start 86.614 78.74) (end 92.795 78.74) (width 0.5) (layer "B.Cu") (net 4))
 (segment (start 92.795 78.74) (end 94.9115 80.8565) (width 0.5) (layer "B.Cu") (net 4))
 (segment (start 86.614 83.566) (end 83.566 86.614) (width 0.5) (layer "B.Cu") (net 4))
 (segment (start 97.875 83.82) (end 94.9115 80.8565) (width 0.5) (layer "B.Cu") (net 4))
 (segment (start 68.960999 83.184999) (end 67.056 83.184999) (width 0.5) (layer "B.Cu") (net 4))
 (segment (start 136.144 83.185) (end 132.207 87.122) (width 0.5) (layer "B.Cu") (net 6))
 (segment (start 109.22 80.01) (end 113.11 80.01) (width 0.5) (layer "B.Cu") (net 6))
 (segment (start 103.59 83.82) (end 105.41 83.82) (width 0.5) (layer "B.Cu") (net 6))
 (segment (start 122.508 87.122) (end 116.586 81.2) (width 0.5) (layer "B.Cu") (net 6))
 (segment (start 113.11 80.01) (end 114.3 81.2) (width 0.5) (layer "B.Cu") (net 6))
 (segment (start 105.41 83.82) (end 109.22 80.01) (width 0.5) (layer "B.Cu") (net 6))
 (segment (start 116.586 81.2) (end 114.3 81.2) (width 0.5) (layer "B.Cu") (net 6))
 (segment (start 132.207 87.122) (end 122.508 87.122) (width 0.5) (layer "B.Cu") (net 6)))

